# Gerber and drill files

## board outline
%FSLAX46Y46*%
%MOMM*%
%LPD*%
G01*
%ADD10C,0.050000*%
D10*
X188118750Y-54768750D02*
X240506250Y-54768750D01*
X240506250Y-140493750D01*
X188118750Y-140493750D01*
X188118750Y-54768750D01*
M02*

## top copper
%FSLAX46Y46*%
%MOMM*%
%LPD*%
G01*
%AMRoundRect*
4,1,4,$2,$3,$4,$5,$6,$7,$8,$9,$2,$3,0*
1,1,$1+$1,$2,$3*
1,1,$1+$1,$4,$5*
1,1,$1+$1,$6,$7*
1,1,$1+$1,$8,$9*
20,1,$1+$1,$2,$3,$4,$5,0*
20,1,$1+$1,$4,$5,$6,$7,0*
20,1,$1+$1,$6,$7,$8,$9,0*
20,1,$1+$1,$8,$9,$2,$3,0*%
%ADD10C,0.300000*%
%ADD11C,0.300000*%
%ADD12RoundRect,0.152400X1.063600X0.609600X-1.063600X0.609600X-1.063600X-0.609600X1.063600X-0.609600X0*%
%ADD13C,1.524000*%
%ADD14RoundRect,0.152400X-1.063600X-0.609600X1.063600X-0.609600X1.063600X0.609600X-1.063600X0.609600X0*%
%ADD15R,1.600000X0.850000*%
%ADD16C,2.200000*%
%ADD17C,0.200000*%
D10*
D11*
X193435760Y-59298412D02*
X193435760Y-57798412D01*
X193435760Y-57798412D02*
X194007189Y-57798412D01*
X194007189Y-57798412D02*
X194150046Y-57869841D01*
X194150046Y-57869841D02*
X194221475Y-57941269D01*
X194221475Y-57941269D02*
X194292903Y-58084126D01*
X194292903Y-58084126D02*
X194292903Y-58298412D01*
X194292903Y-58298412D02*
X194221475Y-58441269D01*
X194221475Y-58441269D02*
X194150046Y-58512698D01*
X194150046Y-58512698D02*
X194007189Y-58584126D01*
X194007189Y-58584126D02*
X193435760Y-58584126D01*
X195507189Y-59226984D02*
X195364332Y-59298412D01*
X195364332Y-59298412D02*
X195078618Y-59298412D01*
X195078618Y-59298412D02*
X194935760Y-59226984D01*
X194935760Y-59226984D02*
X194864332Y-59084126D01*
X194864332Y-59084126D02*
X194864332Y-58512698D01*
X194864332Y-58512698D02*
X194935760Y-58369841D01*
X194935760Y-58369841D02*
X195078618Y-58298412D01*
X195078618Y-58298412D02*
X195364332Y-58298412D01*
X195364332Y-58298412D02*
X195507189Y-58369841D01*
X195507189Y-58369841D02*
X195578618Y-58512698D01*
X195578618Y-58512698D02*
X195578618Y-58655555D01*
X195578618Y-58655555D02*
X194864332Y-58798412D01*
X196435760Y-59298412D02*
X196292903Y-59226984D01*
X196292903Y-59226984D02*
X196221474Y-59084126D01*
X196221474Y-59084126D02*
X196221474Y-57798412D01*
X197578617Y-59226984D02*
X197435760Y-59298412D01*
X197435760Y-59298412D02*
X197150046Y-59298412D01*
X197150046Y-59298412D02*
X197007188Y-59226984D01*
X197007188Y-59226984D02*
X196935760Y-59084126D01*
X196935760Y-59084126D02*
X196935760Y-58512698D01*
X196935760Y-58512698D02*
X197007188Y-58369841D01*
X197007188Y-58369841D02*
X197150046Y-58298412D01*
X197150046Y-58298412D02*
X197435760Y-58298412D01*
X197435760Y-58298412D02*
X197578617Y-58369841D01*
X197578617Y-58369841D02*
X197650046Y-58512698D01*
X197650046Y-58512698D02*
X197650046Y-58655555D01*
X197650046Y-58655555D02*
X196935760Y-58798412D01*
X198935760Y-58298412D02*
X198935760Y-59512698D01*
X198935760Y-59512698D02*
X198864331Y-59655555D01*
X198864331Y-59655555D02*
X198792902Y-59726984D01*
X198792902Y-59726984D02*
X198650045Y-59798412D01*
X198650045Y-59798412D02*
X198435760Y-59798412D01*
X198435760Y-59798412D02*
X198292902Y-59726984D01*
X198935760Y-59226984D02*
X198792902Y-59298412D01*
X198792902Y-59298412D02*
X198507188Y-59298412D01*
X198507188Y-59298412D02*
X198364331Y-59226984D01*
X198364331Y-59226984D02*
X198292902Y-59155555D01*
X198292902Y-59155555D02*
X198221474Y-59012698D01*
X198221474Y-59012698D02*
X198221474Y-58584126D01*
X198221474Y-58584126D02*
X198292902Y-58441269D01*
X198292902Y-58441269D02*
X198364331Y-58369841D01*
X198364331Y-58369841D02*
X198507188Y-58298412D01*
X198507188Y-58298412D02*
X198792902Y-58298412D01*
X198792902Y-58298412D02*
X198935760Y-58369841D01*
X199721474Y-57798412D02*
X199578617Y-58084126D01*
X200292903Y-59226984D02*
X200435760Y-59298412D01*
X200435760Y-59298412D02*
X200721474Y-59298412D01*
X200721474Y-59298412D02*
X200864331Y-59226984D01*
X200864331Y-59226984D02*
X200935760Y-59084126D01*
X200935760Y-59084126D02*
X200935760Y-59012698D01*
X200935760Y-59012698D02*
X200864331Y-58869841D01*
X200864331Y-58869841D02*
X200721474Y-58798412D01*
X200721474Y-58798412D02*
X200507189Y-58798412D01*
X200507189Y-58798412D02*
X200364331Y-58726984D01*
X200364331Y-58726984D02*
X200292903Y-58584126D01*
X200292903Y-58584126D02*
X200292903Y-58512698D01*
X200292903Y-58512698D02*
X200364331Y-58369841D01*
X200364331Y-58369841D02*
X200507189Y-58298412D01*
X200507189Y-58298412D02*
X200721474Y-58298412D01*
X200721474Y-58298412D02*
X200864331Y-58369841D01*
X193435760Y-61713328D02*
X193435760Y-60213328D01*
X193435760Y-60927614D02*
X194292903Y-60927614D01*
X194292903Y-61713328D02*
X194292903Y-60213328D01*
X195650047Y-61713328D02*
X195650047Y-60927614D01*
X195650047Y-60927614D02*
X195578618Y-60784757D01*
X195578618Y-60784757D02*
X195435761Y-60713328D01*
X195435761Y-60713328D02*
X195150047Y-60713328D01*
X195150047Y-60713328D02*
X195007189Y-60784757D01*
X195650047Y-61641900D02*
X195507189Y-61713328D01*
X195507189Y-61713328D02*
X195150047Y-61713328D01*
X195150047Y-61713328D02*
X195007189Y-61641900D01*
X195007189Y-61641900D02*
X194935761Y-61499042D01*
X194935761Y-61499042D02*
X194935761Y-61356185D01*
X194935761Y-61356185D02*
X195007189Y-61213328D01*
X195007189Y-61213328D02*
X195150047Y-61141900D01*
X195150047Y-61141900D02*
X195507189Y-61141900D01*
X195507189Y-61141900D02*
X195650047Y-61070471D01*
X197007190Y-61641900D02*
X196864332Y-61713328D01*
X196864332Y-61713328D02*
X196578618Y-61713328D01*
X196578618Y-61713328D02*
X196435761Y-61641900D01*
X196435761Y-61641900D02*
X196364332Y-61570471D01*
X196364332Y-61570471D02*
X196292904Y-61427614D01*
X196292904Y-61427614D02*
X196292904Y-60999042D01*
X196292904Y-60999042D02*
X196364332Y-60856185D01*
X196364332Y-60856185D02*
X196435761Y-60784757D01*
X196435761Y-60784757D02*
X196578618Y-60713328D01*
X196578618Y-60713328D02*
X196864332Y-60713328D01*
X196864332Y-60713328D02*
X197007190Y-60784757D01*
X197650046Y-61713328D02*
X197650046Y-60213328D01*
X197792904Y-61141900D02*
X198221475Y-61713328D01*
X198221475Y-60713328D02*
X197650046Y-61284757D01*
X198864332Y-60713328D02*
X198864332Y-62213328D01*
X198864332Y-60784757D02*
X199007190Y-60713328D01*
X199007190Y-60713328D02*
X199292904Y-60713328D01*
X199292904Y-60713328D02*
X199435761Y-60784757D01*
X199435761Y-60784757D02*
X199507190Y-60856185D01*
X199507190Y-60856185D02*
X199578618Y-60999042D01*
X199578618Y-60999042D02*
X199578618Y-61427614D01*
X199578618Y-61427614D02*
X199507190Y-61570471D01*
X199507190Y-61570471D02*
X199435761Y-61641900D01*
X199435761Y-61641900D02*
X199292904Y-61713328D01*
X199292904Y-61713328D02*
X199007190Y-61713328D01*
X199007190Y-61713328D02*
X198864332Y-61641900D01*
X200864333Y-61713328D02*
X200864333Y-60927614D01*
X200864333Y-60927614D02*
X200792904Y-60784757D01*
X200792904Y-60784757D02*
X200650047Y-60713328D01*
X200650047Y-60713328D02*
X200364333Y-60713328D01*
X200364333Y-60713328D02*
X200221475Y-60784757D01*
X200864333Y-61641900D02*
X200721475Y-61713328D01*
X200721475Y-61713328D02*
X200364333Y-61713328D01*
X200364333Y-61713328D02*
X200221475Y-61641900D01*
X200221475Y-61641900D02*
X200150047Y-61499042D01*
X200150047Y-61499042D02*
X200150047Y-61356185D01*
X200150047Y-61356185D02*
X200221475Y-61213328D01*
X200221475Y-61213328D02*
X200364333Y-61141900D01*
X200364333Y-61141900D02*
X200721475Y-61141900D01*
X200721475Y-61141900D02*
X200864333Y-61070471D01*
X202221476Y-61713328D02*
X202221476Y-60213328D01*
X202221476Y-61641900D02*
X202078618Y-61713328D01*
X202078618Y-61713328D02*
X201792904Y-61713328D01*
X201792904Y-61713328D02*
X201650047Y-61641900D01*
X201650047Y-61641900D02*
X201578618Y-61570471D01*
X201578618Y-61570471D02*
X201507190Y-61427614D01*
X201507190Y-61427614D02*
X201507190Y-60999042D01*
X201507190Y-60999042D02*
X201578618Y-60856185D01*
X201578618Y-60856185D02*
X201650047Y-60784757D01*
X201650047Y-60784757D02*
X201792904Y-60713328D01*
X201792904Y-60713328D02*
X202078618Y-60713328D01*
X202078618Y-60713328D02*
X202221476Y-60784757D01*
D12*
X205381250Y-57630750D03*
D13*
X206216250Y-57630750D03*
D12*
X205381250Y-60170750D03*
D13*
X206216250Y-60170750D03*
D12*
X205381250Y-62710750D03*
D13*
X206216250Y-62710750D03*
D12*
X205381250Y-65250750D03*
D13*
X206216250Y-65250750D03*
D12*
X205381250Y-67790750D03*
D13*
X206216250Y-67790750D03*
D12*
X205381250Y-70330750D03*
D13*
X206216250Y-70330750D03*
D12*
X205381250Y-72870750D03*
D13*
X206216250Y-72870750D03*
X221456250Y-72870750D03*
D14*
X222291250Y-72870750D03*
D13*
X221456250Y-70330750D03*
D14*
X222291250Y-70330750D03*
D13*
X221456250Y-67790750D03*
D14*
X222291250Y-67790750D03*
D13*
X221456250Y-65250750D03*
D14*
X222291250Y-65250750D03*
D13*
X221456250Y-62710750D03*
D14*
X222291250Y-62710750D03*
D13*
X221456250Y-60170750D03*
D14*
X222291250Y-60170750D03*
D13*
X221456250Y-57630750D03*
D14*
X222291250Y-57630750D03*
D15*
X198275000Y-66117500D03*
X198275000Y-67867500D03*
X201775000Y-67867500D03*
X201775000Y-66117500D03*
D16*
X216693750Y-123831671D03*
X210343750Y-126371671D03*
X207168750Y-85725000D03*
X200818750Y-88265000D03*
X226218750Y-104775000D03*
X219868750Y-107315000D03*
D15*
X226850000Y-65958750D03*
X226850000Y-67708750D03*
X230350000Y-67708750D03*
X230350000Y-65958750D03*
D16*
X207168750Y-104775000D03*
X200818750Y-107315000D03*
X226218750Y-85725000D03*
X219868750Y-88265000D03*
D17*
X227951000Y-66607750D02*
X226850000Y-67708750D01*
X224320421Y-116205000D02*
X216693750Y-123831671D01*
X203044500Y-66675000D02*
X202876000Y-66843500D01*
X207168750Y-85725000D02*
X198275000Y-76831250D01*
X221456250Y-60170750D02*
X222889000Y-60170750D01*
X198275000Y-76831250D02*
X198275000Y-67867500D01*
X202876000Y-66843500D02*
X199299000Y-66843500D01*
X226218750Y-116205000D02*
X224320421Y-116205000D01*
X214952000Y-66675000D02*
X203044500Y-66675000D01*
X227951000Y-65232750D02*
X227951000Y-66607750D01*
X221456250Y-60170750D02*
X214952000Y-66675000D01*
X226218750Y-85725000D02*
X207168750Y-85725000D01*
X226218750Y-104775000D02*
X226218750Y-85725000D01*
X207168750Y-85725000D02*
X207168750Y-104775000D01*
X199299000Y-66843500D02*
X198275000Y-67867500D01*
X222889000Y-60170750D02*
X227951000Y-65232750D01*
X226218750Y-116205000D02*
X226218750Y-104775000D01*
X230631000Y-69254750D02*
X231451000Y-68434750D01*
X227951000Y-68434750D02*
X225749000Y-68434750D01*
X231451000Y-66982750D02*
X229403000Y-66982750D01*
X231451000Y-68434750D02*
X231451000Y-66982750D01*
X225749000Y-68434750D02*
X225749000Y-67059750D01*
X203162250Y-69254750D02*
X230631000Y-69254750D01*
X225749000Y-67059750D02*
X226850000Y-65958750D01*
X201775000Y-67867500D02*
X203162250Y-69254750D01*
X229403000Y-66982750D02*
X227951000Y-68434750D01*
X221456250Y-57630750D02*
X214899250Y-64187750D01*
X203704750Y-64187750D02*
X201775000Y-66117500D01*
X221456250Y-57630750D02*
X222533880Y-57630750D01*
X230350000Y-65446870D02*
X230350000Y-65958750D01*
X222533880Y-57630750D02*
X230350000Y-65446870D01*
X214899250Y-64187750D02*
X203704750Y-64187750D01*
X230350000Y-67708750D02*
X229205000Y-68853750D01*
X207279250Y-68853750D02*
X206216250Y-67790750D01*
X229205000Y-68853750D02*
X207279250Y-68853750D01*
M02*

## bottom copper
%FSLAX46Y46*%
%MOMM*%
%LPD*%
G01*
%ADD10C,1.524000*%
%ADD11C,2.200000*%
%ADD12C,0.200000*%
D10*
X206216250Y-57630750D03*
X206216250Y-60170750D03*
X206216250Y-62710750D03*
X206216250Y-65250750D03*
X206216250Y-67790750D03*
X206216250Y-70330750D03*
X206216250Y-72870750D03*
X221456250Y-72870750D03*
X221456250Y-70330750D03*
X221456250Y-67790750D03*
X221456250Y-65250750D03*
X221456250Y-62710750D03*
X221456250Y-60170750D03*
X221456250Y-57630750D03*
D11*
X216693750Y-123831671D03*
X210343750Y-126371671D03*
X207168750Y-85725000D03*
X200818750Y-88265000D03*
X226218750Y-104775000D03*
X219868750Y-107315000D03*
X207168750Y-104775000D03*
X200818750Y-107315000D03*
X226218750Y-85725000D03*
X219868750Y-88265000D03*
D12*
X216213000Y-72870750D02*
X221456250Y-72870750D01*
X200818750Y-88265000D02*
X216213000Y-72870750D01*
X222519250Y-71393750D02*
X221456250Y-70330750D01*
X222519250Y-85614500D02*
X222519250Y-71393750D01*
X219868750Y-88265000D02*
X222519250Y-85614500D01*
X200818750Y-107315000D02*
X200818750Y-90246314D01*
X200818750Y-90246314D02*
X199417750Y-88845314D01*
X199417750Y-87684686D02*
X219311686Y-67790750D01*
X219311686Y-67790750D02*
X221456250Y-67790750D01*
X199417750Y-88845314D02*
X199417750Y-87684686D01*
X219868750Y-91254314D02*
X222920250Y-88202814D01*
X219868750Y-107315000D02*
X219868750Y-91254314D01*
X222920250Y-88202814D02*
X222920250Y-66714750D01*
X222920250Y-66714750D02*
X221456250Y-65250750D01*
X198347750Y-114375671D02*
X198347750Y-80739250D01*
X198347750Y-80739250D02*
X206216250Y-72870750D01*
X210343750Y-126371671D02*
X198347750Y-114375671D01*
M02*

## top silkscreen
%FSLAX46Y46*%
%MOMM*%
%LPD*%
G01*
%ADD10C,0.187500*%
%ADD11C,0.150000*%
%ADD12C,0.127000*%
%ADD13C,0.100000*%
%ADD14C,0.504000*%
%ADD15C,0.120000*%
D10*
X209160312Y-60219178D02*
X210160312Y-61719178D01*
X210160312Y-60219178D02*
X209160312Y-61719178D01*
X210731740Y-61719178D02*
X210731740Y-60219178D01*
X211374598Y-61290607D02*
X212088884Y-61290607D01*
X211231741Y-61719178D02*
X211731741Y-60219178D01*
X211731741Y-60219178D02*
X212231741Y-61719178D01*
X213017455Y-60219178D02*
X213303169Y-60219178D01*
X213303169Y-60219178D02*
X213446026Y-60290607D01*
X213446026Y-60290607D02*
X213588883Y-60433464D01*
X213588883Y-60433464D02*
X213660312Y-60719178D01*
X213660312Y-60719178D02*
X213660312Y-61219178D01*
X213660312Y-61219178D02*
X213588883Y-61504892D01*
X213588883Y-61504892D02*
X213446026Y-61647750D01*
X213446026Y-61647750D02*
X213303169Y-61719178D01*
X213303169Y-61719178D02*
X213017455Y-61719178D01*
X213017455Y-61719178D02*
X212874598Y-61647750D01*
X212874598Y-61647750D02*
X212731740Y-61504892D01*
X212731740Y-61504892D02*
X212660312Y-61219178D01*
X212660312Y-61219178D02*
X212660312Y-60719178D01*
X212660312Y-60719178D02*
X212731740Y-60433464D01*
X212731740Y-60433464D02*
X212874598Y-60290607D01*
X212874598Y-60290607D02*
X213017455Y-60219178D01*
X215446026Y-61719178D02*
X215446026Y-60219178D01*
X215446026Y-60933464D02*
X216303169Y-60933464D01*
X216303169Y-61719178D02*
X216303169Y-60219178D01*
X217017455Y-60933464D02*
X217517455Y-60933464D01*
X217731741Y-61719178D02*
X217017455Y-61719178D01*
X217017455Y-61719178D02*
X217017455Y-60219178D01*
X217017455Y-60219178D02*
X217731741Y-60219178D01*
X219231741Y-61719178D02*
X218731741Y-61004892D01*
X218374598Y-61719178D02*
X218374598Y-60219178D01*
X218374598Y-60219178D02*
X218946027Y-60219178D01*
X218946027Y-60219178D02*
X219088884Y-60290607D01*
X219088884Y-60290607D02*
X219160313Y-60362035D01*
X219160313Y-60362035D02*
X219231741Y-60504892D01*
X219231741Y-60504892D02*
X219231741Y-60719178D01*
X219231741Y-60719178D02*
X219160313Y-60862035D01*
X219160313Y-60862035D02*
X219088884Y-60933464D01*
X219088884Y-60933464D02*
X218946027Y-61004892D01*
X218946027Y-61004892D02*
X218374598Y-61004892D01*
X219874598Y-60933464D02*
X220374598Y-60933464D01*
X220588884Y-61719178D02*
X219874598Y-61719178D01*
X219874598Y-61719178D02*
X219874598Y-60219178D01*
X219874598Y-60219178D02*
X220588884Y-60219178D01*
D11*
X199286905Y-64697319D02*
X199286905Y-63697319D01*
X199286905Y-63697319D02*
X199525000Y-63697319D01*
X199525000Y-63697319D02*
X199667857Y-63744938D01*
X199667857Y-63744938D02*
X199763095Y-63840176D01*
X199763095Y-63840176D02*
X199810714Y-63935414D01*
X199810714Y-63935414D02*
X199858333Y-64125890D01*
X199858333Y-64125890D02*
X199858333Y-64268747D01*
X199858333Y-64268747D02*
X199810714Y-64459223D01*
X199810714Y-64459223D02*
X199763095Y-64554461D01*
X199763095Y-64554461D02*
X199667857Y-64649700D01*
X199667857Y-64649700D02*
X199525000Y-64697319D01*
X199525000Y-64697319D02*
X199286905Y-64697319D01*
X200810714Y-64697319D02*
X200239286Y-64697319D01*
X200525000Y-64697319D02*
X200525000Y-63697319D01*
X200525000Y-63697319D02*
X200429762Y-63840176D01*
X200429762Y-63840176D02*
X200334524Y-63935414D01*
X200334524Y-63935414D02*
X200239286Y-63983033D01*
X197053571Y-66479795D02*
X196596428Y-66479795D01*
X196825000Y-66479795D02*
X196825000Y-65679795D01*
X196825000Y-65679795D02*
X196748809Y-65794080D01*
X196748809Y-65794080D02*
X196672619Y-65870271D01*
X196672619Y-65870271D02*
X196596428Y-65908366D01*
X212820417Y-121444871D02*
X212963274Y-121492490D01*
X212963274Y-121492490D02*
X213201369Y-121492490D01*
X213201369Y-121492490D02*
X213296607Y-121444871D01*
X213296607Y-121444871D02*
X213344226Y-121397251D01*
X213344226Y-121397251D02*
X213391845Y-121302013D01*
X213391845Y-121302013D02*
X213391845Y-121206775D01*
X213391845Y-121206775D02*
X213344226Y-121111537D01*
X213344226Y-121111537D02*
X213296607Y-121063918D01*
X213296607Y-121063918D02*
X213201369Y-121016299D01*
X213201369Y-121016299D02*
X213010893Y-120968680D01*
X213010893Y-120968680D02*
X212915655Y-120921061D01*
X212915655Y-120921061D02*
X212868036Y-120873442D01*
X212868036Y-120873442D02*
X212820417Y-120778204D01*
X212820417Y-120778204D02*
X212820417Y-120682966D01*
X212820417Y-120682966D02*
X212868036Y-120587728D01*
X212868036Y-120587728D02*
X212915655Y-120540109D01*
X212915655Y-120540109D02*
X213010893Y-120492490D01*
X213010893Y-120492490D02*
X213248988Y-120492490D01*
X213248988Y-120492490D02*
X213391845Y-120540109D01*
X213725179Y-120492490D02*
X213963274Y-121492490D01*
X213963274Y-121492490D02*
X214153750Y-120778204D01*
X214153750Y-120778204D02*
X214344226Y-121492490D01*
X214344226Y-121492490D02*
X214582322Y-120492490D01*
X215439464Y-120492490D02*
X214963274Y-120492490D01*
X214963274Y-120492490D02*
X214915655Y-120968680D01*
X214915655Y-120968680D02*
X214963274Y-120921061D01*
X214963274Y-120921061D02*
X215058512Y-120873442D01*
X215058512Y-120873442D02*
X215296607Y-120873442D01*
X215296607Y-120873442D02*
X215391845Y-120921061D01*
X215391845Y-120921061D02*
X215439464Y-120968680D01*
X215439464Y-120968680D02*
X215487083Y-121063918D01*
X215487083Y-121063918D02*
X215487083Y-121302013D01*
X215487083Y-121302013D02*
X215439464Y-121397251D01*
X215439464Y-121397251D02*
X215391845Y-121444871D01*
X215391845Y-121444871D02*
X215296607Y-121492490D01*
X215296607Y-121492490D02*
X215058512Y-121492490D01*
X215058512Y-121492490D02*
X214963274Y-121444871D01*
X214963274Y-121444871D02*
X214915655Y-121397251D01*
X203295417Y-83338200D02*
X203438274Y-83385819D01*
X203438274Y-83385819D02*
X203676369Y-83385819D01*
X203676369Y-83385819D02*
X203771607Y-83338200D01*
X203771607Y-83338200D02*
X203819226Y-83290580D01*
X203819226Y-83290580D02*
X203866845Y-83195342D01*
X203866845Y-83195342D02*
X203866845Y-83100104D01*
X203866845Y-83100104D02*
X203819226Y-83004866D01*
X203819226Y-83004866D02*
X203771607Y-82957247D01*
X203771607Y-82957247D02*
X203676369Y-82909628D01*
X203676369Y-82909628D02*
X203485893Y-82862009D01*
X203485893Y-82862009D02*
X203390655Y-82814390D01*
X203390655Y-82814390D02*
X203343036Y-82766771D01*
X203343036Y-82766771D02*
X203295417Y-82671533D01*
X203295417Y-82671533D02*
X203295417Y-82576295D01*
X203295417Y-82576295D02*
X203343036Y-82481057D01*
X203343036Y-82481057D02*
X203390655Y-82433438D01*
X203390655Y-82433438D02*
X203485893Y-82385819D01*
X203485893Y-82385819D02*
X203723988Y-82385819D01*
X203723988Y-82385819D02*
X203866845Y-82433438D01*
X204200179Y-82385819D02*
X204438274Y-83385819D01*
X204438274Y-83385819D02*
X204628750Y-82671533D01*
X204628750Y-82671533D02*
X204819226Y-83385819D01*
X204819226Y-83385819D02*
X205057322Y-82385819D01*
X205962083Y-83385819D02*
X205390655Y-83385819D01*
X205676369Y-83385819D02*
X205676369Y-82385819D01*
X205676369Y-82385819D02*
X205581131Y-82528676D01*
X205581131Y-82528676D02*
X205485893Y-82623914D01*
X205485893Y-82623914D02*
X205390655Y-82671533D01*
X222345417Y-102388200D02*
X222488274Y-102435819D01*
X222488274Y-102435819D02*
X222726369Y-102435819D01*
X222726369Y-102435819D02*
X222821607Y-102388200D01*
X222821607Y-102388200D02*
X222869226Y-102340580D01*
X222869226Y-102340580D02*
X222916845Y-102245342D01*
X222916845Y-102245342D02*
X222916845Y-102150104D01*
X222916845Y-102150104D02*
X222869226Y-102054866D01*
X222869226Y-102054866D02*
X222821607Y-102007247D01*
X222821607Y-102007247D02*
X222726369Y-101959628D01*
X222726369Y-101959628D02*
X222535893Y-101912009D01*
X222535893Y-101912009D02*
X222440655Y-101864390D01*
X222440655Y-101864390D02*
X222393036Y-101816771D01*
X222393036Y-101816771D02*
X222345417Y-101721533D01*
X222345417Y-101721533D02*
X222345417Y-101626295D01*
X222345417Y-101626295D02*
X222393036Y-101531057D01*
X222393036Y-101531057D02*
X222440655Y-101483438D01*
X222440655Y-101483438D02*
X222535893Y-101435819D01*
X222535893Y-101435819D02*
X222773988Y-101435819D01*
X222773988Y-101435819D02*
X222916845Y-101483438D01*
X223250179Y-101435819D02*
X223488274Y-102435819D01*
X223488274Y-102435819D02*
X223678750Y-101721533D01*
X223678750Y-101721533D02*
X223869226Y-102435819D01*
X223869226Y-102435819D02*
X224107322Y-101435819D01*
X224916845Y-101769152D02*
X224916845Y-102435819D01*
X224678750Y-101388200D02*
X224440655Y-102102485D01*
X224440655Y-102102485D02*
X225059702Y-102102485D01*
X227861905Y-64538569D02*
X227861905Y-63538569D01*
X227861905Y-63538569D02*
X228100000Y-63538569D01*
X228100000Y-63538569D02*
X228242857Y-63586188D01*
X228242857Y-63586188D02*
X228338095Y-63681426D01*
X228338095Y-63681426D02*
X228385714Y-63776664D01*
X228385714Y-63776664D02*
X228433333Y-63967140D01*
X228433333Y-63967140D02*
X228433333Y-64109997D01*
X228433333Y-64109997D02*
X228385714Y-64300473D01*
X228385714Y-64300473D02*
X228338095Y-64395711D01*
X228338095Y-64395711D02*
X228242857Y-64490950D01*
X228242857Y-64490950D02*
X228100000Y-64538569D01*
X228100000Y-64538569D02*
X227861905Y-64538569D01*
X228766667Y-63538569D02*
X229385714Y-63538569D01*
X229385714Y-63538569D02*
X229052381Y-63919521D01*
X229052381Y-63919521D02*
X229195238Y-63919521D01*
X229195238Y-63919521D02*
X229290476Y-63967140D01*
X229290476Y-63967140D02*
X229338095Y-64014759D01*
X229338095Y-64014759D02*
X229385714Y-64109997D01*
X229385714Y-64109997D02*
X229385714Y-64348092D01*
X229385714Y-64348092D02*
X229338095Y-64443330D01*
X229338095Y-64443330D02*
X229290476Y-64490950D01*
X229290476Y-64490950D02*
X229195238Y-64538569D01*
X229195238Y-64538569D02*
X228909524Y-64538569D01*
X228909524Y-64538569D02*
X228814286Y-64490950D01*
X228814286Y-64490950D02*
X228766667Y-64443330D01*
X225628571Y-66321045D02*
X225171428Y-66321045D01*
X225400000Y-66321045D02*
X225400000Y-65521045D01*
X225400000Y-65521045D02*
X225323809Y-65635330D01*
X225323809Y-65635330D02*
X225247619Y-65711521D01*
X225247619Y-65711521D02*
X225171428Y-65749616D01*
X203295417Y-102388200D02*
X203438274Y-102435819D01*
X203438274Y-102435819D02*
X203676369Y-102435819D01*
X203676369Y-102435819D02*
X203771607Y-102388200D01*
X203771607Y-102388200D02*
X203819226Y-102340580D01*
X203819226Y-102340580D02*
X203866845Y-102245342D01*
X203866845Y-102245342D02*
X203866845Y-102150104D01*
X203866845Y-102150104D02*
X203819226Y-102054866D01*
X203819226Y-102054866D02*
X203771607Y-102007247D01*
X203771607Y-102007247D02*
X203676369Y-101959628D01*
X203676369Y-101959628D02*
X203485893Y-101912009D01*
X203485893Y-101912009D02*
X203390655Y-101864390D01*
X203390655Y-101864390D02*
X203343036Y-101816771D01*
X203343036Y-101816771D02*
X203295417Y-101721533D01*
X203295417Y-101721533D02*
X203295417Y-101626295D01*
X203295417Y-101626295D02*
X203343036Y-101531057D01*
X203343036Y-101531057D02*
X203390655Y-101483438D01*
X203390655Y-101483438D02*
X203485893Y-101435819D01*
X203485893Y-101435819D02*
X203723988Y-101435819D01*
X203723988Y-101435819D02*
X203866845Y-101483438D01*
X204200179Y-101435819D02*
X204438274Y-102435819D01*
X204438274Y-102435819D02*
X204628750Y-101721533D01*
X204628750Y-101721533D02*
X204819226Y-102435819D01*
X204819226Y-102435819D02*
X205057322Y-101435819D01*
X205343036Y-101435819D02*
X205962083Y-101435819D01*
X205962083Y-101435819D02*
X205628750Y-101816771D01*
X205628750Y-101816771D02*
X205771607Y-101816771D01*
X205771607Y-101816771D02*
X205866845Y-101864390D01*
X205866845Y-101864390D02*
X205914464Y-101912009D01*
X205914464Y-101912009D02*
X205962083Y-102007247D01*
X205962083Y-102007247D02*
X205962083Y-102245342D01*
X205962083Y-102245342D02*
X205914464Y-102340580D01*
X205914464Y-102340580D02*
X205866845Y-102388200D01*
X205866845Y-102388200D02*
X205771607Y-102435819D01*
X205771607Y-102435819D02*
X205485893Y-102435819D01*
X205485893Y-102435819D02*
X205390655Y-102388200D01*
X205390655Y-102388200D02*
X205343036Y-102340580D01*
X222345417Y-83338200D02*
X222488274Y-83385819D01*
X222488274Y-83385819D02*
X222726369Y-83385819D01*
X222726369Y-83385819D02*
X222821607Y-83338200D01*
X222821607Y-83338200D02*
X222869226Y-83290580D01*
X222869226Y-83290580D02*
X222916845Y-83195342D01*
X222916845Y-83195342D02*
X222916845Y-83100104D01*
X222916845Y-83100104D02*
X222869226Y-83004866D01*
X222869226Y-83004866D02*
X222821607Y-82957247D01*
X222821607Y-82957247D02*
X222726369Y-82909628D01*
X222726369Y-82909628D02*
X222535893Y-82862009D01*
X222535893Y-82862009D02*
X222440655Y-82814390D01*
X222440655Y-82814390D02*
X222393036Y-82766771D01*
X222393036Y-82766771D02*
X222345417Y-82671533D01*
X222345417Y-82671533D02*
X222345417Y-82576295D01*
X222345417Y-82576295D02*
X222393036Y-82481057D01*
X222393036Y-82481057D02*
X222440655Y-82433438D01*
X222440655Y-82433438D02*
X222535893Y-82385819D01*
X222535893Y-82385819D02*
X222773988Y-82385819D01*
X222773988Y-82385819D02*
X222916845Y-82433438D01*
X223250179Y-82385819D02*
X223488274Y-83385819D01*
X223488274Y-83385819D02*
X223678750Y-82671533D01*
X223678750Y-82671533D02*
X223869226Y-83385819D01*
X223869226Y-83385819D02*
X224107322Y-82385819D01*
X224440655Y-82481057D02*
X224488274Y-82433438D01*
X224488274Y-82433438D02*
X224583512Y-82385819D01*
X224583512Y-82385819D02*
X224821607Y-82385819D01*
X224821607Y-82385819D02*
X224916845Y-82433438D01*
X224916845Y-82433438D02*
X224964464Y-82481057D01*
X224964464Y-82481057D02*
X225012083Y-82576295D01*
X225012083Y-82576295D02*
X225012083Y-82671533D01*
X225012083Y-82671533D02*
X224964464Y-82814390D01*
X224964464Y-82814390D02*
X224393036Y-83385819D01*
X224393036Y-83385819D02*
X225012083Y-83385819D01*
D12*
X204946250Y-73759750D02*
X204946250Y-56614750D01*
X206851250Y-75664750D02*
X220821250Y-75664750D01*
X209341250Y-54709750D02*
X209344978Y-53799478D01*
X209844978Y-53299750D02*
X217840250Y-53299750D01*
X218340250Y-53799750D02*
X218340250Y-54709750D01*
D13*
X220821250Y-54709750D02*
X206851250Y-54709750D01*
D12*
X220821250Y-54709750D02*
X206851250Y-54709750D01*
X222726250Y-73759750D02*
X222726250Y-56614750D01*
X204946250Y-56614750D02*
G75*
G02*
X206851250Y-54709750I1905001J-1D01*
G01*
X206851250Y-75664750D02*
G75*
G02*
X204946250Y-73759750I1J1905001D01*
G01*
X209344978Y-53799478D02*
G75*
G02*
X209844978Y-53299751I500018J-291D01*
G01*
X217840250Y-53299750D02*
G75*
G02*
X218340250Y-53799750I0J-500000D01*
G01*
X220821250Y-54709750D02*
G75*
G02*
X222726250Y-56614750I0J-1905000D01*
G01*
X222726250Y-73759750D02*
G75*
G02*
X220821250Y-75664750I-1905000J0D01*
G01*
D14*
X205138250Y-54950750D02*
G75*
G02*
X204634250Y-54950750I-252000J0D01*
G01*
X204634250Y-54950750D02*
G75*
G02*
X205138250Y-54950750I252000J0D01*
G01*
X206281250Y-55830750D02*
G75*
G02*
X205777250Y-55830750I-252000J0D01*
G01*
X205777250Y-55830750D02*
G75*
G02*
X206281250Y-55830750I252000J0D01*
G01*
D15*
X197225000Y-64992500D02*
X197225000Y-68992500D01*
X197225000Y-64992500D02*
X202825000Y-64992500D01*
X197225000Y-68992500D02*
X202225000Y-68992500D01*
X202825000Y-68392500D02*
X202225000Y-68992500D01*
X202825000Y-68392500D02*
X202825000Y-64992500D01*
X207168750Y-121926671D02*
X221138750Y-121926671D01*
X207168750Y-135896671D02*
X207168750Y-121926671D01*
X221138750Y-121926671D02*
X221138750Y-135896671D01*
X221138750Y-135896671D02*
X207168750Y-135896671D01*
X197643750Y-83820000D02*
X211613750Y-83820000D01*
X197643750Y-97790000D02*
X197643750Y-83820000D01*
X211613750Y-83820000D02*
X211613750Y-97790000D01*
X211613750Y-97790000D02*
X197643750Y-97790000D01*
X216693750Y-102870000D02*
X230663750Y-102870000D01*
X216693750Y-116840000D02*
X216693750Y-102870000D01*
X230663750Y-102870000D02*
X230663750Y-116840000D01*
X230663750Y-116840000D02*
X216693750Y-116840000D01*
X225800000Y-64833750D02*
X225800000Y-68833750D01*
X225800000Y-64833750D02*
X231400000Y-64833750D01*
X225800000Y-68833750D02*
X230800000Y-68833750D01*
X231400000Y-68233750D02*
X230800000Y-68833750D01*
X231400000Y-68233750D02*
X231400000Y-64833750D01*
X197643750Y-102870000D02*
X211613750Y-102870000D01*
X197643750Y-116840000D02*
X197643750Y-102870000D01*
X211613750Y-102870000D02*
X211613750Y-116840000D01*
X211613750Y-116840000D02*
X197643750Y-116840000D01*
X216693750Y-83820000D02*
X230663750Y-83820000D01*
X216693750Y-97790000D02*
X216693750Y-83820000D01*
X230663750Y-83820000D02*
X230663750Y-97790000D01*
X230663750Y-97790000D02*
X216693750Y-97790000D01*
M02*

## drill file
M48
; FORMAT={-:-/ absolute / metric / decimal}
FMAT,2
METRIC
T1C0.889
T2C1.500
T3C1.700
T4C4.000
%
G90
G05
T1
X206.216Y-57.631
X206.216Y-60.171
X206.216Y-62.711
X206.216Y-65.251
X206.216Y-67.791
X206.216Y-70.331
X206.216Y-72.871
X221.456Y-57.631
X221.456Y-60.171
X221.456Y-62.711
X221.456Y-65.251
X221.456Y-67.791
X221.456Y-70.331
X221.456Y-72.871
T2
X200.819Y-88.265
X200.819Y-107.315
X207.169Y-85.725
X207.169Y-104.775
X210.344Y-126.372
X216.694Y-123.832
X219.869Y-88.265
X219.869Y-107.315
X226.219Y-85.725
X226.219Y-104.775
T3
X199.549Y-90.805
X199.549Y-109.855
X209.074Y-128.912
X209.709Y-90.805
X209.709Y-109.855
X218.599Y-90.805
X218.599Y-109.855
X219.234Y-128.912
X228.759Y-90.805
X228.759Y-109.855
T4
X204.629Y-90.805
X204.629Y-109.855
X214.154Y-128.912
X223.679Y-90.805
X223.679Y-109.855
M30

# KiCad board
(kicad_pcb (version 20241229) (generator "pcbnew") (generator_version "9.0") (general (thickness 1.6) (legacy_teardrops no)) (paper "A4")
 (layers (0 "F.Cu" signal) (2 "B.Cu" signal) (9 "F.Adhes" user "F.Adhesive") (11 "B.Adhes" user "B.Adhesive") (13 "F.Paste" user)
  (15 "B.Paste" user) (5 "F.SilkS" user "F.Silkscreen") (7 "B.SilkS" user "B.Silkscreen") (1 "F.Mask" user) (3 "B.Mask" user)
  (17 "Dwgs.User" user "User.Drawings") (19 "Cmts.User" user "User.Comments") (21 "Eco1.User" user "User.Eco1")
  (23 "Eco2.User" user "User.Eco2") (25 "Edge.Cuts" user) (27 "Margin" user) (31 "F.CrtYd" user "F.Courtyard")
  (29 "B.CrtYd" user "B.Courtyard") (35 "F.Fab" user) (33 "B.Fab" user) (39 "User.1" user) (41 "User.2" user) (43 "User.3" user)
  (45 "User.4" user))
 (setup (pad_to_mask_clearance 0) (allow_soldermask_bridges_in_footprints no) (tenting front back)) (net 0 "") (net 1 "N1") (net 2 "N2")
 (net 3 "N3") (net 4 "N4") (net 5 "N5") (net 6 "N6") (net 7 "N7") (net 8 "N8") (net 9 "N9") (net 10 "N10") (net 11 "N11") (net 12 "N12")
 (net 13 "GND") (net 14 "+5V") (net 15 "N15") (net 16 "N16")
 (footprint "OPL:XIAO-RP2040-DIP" (layer "F.Cu") (at 213.83625 65.25075)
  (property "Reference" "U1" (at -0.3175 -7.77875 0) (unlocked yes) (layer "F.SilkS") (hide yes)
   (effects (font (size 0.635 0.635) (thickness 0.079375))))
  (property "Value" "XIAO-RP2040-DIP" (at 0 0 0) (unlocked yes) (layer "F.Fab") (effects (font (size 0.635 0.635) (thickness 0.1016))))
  (fp_line (start -8.89 8.509) (end -8.89 -8.636) (stroke (width 0.127) (type solid)) (layer "F.SilkS"))
  (fp_line (start -6.985 10.414) (end 6.985 10.414) (stroke (width 0.127) (type solid)) (layer "F.SilkS"))
  (fp_line (start -4.495 -10.541) (end -4.491272 -11.451272) (stroke (width 0.127) (type solid)) (layer "F.SilkS"))
  (fp_line (start -3.991272 -11.951) (end 4.004 -11.951) (stroke (width 0.127) (type solid)) (layer "F.SilkS"))
  (fp_line (start 4.504 -11.451) (end 4.504 -10.541) (stroke (width 0.127) (type solid)) (layer "F.SilkS"))
  (fp_line (start 6.985 -10.541) (end -6.985 -10.541) (stroke (width 0.1) (type solid)) (layer "F.SilkS"))
  (fp_line (start 6.985 -10.541) (end -6.985 -10.541) (stroke (width 0.127) (type solid)) (layer "F.SilkS"))
  (fp_line (start 8.89 8.509) (end 8.89 -8.636) (stroke (width 0.127) (type solid)) (layer "F.SilkS"))
  (fp_arc (start -8.89 -8.636) (mid -8.332038 -9.983038) (end -6.985 -10.541) (stroke (width 0.127) (type solid)) (layer "F.SilkS"))
  (fp_arc (start -6.985 10.414) (mid -8.332038 9.856038) (end -8.89 8.509) (stroke (width 0.127) (type solid)) (layer "F.SilkS"))
  (fp_arc (start -4.491272 -11.451272) (mid -4.344728 -11.80464) (end -3.991272 -11.951) (stroke (width 0.127) (type default))
   (layer "F.SilkS"))
  (fp_arc (start 4.004 -11.951) (mid 4.357553 -11.804553) (end 4.504 -11.451) (stroke (width 0.127) (type default)) (layer "F.SilkS"))
  (fp_arc (start 6.985 -10.541) (mid 8.332038 -9.983038) (end 8.89 -8.636) (stroke (width 0.127) (type solid)) (layer "F.SilkS"))
  (fp_arc (start 8.89 8.509) (mid 8.332038 9.856038) (end 6.985 10.414) (stroke (width 0.127) (type solid)) (layer "F.SilkS"))
  (fp_circle (center -8.95 -10.3) (end -8.95 -10.554) (stroke (width 0.5) (type solid)) (fill yes) (layer "F.SilkS"))
  (fp_circle (center -7.807 -9.42) (end -7.807 -9.674) (stroke (width 0.5) (type solid)) (fill yes) (layer "F.SilkS"))
  (pad "1" smd roundrect (at -8.455 -7.62 180) (size 2.432 1.524) (layers "F.Cu" "F.Mask") (roundrect_rratio 0.1) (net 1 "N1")
   (thermal_bridge_angle 45))
  (pad "1" thru_hole circle (at -7.62 -7.62 180) (size 1.524 1.524) (drill 0.889) (layers "*.Cu" "*.Mask") (remove_unused_layers no)
   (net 1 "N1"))
  (pad "2" smd roundrect (at -8.455 -5.08 180) (size 2.432 1.524) (layers "F.Cu" "F.Mask") (roundrect_rratio 0.1) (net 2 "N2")
   (thermal_bridge_angle 45))
  (pad "2" thru_hole circle (at -7.62 -5.08 180) (size 1.524 1.524) (drill 0.889) (layers "*.Cu" "*.Mask") (remove_unused_layers no)
   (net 2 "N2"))
  (pad "3" smd roundrect (at -8.455 -2.54 180) (size 2.432 1.524) (layers "F.Cu" "F.Mask") (roundrect_rratio 0.1) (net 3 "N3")
   (thermal_bridge_angle 45))
  (pad "3" thru_hole circle (at -7.62 -2.54 180) (size 1.524 1.524) (drill 0.889) (layers "*.Cu" "*.Mask") (remove_unused_layers no)
   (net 3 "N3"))
  (pad "4" smd roundrect (at -8.455 0 180) (size 2.432 1.524) (layers "F.Cu" "F.Mask") (roundrect_rratio 0.1) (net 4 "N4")
   (thermal_bridge_angle 45))
  (pad "4" thru_hole circle (at -7.62 0 180) (size 1.524 1.524) (drill 0.889) (layers "*.Cu" "*.Mask") (remove_unused_layers no)
   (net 4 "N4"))
  (pad "5" smd roundrect (at -8.455 2.54 180) (size 2.432 1.524) (layers "F.Cu" "F.Mask") (roundrect_rratio 0.1) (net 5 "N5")
   (thermal_bridge_angle 45))
  (pad "5" thru_hole circle (at -7.62 2.54 180) (size 1.524 1.524) (drill 0.889) (layers "*.Cu" "*.Mask") (remove_unused_layers no)
   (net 5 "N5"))
  (pad "6" smd roundrect (at -8.455 5.08 180) (size 2.432 1.524) (layers "F.Cu" "F.Mask") (roundrect_rratio 0.1) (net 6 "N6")
   (thermal_bridge_angle 45))
  (pad "6" thru_hole circle (at -7.62 5.08 180) (size 1.524 1.524) (drill 0.889) (layers "*.Cu" "*.Mask") (remove_unused_layers no)
   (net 6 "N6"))
  (pad "7" smd roundrect (at -8.455 7.62 180) (size 2.432 1.524) (layers "F.Cu" "F.Mask") (roundrect_rratio 0.1) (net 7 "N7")
   (thermal_bridge_angle 45))
  (pad "7" thru_hole circle (at -7.62 7.62 180) (size 1.524 1.524) (drill 0.889) (layers "*.Cu" "*.Mask") (remove_unused_layers no)
   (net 7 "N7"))
  (pad "8" thru_hole circle (at 7.62 7.62) (size 1.524 1.524) (drill 0.889) (layers "*.Cu" "*.Mask") (remove_unused_layers no) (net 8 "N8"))
  (pad "8" smd roundrect (at 8.455 7.62) (size 2.432 1.524) (layers "F.Cu" "F.Mask") (roundrect_rratio 0.1) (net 8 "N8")
   (thermal_bridge_angle 45))
  (pad "9" thru_hole circle (at 7.62 5.08) (size 1.524 1.524) (drill 0.889) (layers "*.Cu" "*.Mask") (remove_unused_layers no) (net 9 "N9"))
  (pad "9" smd roundrect (at 8.455 5.08) (size 2.432 1.524) (layers "F.Cu" "F.Mask") (roundrect_rratio 0.1) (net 9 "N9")
   (thermal_bridge_angle 45))
  (pad "10" thru_hole circle (at 7.62 2.54) (size 1.524 1.524) (drill 0.889) (layers "*.Cu" "*.Mask") (remove_unused_layers no)
   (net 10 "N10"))
  (pad "10" smd roundrect (at 8.455 2.54) (size 2.432 1.524) (layers "F.Cu" "F.Mask") (roundrect_rratio 0.1) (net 10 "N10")
   (thermal_bridge_angle 45))
  (pad "11" thru_hole circle (at 7.62 0) (size 1.524 1.524) (drill 0.889) (layers "*.Cu" "*.Mask") (remove_unused_layers no) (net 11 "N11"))
  (pad "11" smd roundrect (at 8.455 0) (size 2.432 1.524) (layers "F.Cu" "F.Mask") (roundrect_rratio 0.1) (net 11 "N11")
   (thermal_bridge_angle 45))
  (pad "12" thru_hole circle (at 7.62 -2.54) (size 1.524 1.524) (drill 0.889) (layers "*.Cu" "*.Mask") (remove_unused_layers no)
   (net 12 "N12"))
  (pad "12" smd roundrect (at 8.455 -2.54) (size 2.432 1.524) (layers "F.Cu" "F.Mask") (roundrect_rratio 0.1) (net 12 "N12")
   (thermal_bridge_angle 45))
  (pad "13" thru_hole circle (at 7.62 -5.08) (size 1.524 1.524) (drill 0.889) (layers "*.Cu" "*.Mask") (remove_unused_layers no)
   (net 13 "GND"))
  (pad "13" smd roundrect (at 8.455 -5.08) (size 2.432 1.524) (layers "F.Cu" "F.Mask") (roundrect_rratio 0.1) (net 13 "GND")
   (thermal_bridge_angle 45))
  (pad "14" thru_hole circle (at 7.62 -7.62) (size 1.524 1.524) (drill 0.889) (layers "*.Cu" "*.Mask") (remove_unused_layers no)
   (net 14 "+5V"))
  (pad "14" smd roundrect (at 8.455 -7.62) (size 2.432 1.524) (layers "F.Cu" "F.Mask") (roundrect_rratio 0.1) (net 14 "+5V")
   (thermal_bridge_angle 45)))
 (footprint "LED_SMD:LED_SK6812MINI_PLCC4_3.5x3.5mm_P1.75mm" (layer "F.Cu") (at 200.025 66.9925)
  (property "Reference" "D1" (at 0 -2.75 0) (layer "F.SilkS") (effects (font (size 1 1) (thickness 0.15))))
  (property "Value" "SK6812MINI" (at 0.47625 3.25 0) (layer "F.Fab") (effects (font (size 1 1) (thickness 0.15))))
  (fp_line (start -2.8 -2) (end -2.8 2) (stroke (width 0.12) (type default)) (layer "F.SilkS"))
  (fp_line (start -2.8 -2) (end 2.8 -2) (stroke (width 0.12) (type solid)) (layer "F.SilkS"))
  (fp_line (start -2.8 2) (end 2.2 2) (stroke (width 0.12) (type solid)) (layer "F.SilkS"))
  (fp_line (start 2.8 1.4) (end 2.2 2) (stroke (width 0.12) (type default)) (layer "F.SilkS"))
  (fp_line (start 2.8 1.4) (end 2.8 -2) (stroke (width 0.12) (type solid)) (layer "F.SilkS"))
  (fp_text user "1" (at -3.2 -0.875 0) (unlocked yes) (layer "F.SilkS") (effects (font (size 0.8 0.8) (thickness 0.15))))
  (pad "1" smd rect (at -1.75 -0.875) (size 1.6 0.85) (layers "F.Cu" "F.Mask" "F.Paste") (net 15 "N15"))
  (pad "2" smd rect (at -1.75 0.875) (size 1.6 0.85) (layers "F.Cu" "F.Mask" "F.Paste") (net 13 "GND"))
  (pad "3" smd rect (at 1.75 0.875) (size 1.6 0.85) (layers "F.Cu" "F.Mask" "F.Paste") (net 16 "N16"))
  (pad "4" smd rect (at 1.75 -0.875) (size 1.6 0.85) (layers "F.Cu" "F.Mask" "F.Paste") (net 14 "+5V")))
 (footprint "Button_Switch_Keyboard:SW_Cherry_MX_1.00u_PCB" (layer "F.Cu") (at 216.69375 123.831671)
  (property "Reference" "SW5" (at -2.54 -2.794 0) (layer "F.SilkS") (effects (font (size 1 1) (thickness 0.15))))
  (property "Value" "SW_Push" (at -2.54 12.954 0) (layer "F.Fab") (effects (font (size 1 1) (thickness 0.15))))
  (fp_line (start -9.525 -1.905) (end 4.445 -1.905) (stroke (width 0.12) (type solid)) (layer "F.SilkS"))
  (fp_line (start -9.525 12.065) (end -9.525 -1.905) (stroke (width 0.12) (type solid)) (layer "F.SilkS"))
  (fp_line (start 4.445 -1.905) (end 4.445 12.065) (stroke (width 0.12) (type solid)) (layer "F.SilkS"))
  (fp_line (start 4.445 12.065) (end -9.525 12.065) (stroke (width 0.12) (type solid)) (layer "F.SilkS"))
  (pad "" np_thru_hole circle (at -7.62 5.08) (size 1.7 1.7) (drill 1.7) (layers "*.Cu" "*.Mask"))
  (pad "" np_thru_hole circle (at -2.54 5.08) (size 4 4) (drill 4) (layers "*.Cu" "*.Mask"))
  (pad "" np_thru_hole circle (at 2.54 5.08) (size 1.7 1.7) (drill 1.7) (layers "*.Cu" "*.Mask"))
  (pad "1" thru_hole circle (at 0 0) (size 2.2 2.2) (drill 1.5) (layers "*.Cu" "*.Mask") (remove_unused_layers no) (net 13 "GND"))
  (pad "2" thru_hole circle (at -6.35 2.54) (size 2.2 2.2) (drill 1.5) (layers "*.Cu" "*.Mask") (remove_unused_layers no) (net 7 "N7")))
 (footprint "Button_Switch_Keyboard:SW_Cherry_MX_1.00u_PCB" (layer "F.Cu") (at 207.16875 85.725)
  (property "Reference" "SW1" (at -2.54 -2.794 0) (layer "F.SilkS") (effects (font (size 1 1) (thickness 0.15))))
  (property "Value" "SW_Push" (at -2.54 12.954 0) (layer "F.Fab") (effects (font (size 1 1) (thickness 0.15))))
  (fp_line (start -9.525 -1.905) (end 4.445 -1.905) (stroke (width 0.12) (type solid)) (layer "F.SilkS"))
  (fp_line (start -9.525 12.065) (end -9.525 -1.905) (stroke (width 0.12) (type solid)) (layer "F.SilkS"))
  (fp_line (start 4.445 -1.905) (end 4.445 12.065) (stroke (width 0.12) (type solid)) (layer "F.SilkS"))
  (fp_line (start 4.445 12.065) (end -9.525 12.065) (stroke (width 0.12) (type solid)) (layer "F.SilkS"))
  (pad "" np_thru_hole circle (at -7.62 5.08) (size 1.7 1.7) (drill 1.7) (layers "*.Cu" "*.Mask"))
  (pad "" np_thru_hole circle (at -2.54 5.08) (size 4 4) (drill 4) (layers "*.Cu" "*.Mask"))
  (pad "" np_thru_hole circle (at 2.54 5.08) (size 1.7 1.7) (drill 1.7) (layers "*.Cu" "*.Mask"))
  (pad "1" thru_hole circle (at 0 0) (size 2.2 2.2) (drill 1.5) (layers "*.Cu" "*.Mask") (remove_unused_layers no) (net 13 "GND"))
  (pad "2" thru_hole circle (at -6.35 2.54) (size 2.2 2.2) (drill 1.5) (layers "*.Cu" "*.Mask") (remove_unused_layers no) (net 8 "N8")))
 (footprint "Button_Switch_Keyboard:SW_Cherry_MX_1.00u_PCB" (layer "F.Cu") (at 226.21875 104.775)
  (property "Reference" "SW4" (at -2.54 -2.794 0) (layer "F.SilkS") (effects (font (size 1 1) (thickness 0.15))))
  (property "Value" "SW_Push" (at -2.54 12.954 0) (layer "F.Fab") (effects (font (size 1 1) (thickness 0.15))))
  (fp_line (start -9.525 -1.905) (end 4.445 -1.905) (stroke (width 0.12) (type solid)) (layer "F.SilkS"))
  (fp_line (start -9.525 12.065) (end -9.525 -1.905) (stroke (width 0.12) (type solid)) (layer "F.SilkS"))
  (fp_line (start 4.445 -1.905) (end 4.445 12.065) (stroke (width 0.12) (type solid)) (layer "F.SilkS"))
  (fp_line (start 4.445 12.065) (end -9.525 12.065) (stroke (width 0.12) (type solid)) (layer "F.SilkS"))
  (pad "" np_thru_hole circle (at -7.62 5.08) (size 1.7 1.7) (drill 1.7) (layers "*.Cu" "*.Mask"))
  (pad "" np_thru_hole circle (at -2.54 5.08) (size 4 4) (drill 4) (layers "*.Cu" "*.Mask"))
  (pad "" np_thru_hole circle (at 2.54 5.08) (size 1.7 1.7) (drill 1.7) (layers "*.Cu" "*.Mask"))
  (pad "1" thru_hole circle (at 0 0) (size 2.2 2.2) (drill 1.5) (layers "*.Cu" "*.Mask") (remove_unused_layers no) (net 13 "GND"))
  (pad "2" thru_hole circle (at -6.35 2.54) (size 2.2 2.2) (drill 1.5) (layers "*.Cu" "*.Mask") (remove_unused_layers no) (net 11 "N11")))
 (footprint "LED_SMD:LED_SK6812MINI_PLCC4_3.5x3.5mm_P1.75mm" (layer "F.Cu") (at 228.6 66.83375)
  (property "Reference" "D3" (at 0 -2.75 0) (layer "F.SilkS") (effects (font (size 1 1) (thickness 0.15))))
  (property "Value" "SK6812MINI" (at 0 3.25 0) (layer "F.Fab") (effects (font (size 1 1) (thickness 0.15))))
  (fp_line (start -2.8 -2) (end -2.8 2) (stroke (width 0.12) (type default)) (layer "F.SilkS"))
  (fp_line (start -2.8 -2) (end 2.8 -2) (stroke (width 0.12) (type solid)) (layer "F.SilkS"))
  (fp_line (start -2.8 2) (end 2.2 2) (stroke (width 0.12) (type solid)) (layer "F.SilkS"))
  (fp_line (start 2.8 1.4) (end 2.2 2) (stroke (width 0.12) (type default)) (layer "F.SilkS"))
  (fp_line (start 2.8 1.4) (end 2.8 -2) (stroke (width 0.12) (type solid)) (layer "F.SilkS"))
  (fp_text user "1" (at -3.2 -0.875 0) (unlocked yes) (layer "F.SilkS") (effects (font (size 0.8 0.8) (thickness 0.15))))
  (pad "1" smd rect (at -1.75 -0.875) (size 1.6 0.85) (layers "F.Cu" "F.Mask" "F.Paste") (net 16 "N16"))
  (pad "2" smd rect (at -1.75 0.875) (size 1.6 0.85) (layers "F.Cu" "F.Mask" "F.Paste") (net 13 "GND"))
  (pad "3" smd rect (at 1.75 0.875) (size 1.6 0.85) (layers "F.Cu" "F.Mask" "F.Paste") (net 5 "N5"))
  (pad "4" smd rect (at 1.75 -0.875) (size 1.6 0.85) (layers "F.Cu" "F.Mask" "F.Paste") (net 14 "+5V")))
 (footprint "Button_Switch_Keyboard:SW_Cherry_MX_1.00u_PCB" (layer "F.Cu") (at 207.16875 104.775)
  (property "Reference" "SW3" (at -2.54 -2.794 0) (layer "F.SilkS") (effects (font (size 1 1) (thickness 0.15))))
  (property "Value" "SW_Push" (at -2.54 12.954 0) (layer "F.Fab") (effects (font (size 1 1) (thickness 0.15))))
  (fp_line (start -9.525 -1.905) (end 4.445 -1.905) (stroke (width 0.12) (type solid)) (layer "F.SilkS"))
  (fp_line (start -9.525 12.065) (end -9.525 -1.905) (stroke (width 0.12) (type solid)) (layer "F.SilkS"))
  (fp_line (start 4.445 -1.905) (end 4.445 12.065) (stroke (width 0.12) (type solid)) (layer "F.SilkS"))
  (fp_line (start 4.445 12.065) (end -9.525 12.065) (stroke (width 0.12) (type solid)) (layer "F.SilkS"))
  (pad "" np_thru_hole circle (at -7.62 5.08) (size 1.7 1.7) (drill 1.7) (layers "*.Cu" "*.Mask"))
  (pad "" np_thru_hole circle (at -2.54 5.08) (size 4 4) (drill 4) (layers "*.Cu" "*.Mask"))
  (pad "" np_thru_hole circle (at 2.54 5.08) (size 1.7 1.7) (drill 1.7) (layers "*.Cu" "*.Mask"))
  (pad "1" thru_hole circle (at 0 0) (size 2.2 2.2) (drill 1.5) (layers "*.Cu" "*.Mask") (remove_unused_layers no) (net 13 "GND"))
  (pad "2" thru_hole circle (at -6.35 2.54) (size 2.2 2.2) (drill 1.5) (layers "*.Cu" "*.Mask") (remove_unused_layers no) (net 10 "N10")))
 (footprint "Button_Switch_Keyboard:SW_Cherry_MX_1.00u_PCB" (layer "F.Cu") (at 226.21875 85.725)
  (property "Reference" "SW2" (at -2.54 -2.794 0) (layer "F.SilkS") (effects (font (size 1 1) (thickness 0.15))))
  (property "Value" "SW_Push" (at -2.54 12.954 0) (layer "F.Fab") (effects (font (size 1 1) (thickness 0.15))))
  (fp_line (start -9.525 -1.905) (end 4.445 -1.905) (stroke (width 0.12) (type solid)) (layer "F.SilkS"))
  (fp_line (start -9.525 12.065) (end -9.525 -1.905) (stroke (width 0.12) (type solid)) (layer "F.SilkS"))
  (fp_line (start 4.445 -1.905) (end 4.445 12.065) (stroke (width 0.12) (type solid)) (layer "F.SilkS"))
  (fp_line (start 4.445 12.065) (end -9.525 12.065) (stroke (width 0.12) (type solid)) (layer "F.SilkS"))
  (pad "" np_thru_hole circle (at -7.62 5.08) (size 1.7 1.7) (drill 1.7) (layers "*.Cu" "*.Mask"))
  (pad "" np_thru_hole circle (at -2.54 5.08) (size 4 4) (drill 4) (layers "*.Cu" "*.Mask"))
  (pad "" np_thru_hole circle (at 2.54 5.08) (size 1.7 1.7) (drill 1.7) (layers "*.Cu" "*.Mask"))
  (pad "1" thru_hole circle (at 0 0) (size 2.2 2.2) (drill 1.5) (layers "*.Cu" "*.Mask") (remove_unused_layers no) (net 13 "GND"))
  (pad "2" thru_hole circle (at -6.35 2.54) (size 2.2 2.2) (drill 1.5) (layers "*.Cu" "*.Mask") (remove_unused_layers no) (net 9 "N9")))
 (gr_rect (start 188.11875 54.76875) (end 240.50625 140.49375) (stroke (width 0.05) (type default)) (fill no) (layer "Edge.Cuts"))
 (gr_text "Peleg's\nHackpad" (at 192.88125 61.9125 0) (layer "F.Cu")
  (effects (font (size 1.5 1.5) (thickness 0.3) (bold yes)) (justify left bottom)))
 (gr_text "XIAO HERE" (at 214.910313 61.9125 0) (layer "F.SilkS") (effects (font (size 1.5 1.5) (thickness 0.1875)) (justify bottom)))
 (segment (start 227.951 66.60775) (end 226.85 67.70875) (width 0.2) (layer "F.Cu") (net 13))
 (segment (start 224.320421 116.205) (end 216.69375 123.831671) (width 0.2) (layer "F.Cu") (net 13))
 (segment (start 203.0445 66.675) (end 202.876 66.8435) (width 0.2) (layer "F.Cu") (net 13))
 (segment (start 207.16875 85.725) (end 198.275 76.83125) (width 0.2) (layer "F.Cu") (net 13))
 (segment (start 221.45625 60.17075) (end 222.889 60.17075) (width 0.2) (layer "F.Cu") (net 13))
 (segment (start 198.275 76.83125) (end 198.275 67.8675) (width 0.2) (layer "F.Cu") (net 13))
 (segment (start 202.876 66.8435) (end 199.299 66.8435) (width 0.2) (layer "F.Cu") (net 13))
 (segment (start 226.21875 116.205) (end 224.320421 116.205) (width 0.2) (layer "F.Cu") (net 13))
 (segment (start 214.952 66.675) (end 203.0445 66.675) (width 0.2) (layer "F.Cu") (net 13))
 (segment (start 227.951 65.23275) (end 227.951 66.60775) (width 0.2) (layer "F.Cu") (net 13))
 (segment (start 221.45625 60.17075) (end 214.952 66.675) (width 0.2) (layer "F.Cu") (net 13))
 (segment (start 226.21875 85.725) (end 207.16875 85.725) (width 0.2) (layer "F.Cu") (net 13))
 (segment (start 226.21875 104.775) (end 226.21875 85.725) (width 0.2) (layer "F.Cu") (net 13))
 (segment (start 207.16875 85.725) (end 207.16875 104.775) (width 0.2) (layer "F.Cu") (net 13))
 (segment (start 199.299 66.8435) (end 198.275 67.8675) (width 0.2) (layer "F.Cu") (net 13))
 (segment (start 222.889 60.17075) (end 227.951 65.23275) (width 0.2) (layer "F.Cu") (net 13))
 (segment (start 226.21875 116.205) (end 226.21875 104.775) (width 0.2) (layer "F.Cu") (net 13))
 (segment (start 230.631 69.25475) (end 231.451 68.43475) (width 0.2) (layer "F.Cu") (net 16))
 (segment (start 227.951 68.43475) (end 225.749 68.43475) (width 0.2) (layer "F.Cu") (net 16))
 (segment (start 231.451 66.98275) (end 229.403 66.98275) (width 0.2) (layer "F.Cu") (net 16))
 (segment (start 231.451 68.43475) (end 231.451 66.98275) (width 0.2) (layer "F.Cu") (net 16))
 (segment (start 225.749 68.43475) (end 225.749 67.05975) (width 0.2) (layer "F.Cu") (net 16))
 (segment (start 203.16225 69.25475) (end 230.631 69.25475) (width 0.2) (layer "F.Cu") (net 16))
 (segment (start 225.749 67.05975) (end 226.85 65.95875) (width 0.2) (layer "F.Cu") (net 16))
 (segment (start 201.775 67.8675) (end 203.16225 69.25475) (width 0.2) (layer "F.Cu") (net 16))
 (segment (start 229.403 66.98275) (end 227.951 68.43475) (width 0.2) (layer "F.Cu") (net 16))
 (segment (start 221.45625 57.63075) (end 214.89925 64.18775) (width 0.2) (layer "F.Cu") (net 14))
 (segment (start 203.70475 64.18775) (end 201.775 66.1175) (width 0.2) (layer "F.Cu") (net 14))
 (segment (start 221.45625 57.63075) (end 222.53388 57.63075) (width 0.2) (layer "F.Cu") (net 14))
 (segment (start 230.35 65.44687) (end 230.35 65.95875) (width 0.2) (layer "F.Cu") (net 14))
 (segment (start 222.53388 57.63075) (end 230.35 65.44687) (width 0.2) (layer "F.Cu") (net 14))
 (segment (start 214.89925 64.18775) (end 203.70475 64.18775) (width 0.2) (layer "F.Cu") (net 14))
 (segment (start 230.35 67.70875) (end 229.205 68.85375) (width 0.2) (layer "F.Cu") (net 5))
 (segment (start 207.27925 68.85375) (end 206.21625 67.79075) (width 0.2) (layer "F.Cu") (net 5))
 (segment (start 229.205 68.85375) (end 207.27925 68.85375) (width 0.2) (layer "F.Cu") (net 5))
 (segment (start 216.213 72.87075) (end 221.45625 72.87075) (width 0.2) (layer "B.Cu") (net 8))
 (segment (start 200.81875 88.265) (end 216.213 72.87075) (width 0.2) (layer "B.Cu") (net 8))
 (segment (start 222.51925 71.39375) (end 221.45625 70.33075) (width 0.2) (layer "B.Cu") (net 9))
 (segment (start 222.51925 85.6145) (end 222.51925 71.39375) (width 0.2) (layer "B.Cu") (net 9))
 (segment (start 219.86875 88.265) (end 222.51925 85.6145) (width 0.2) (layer "B.Cu") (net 9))
 (segment (start 200.81875 107.315) (end 200.81875 90.246314) (width 0.2) (layer "B.Cu") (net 10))
 (segment (start 200.81875 90.246314) (end 199.41775 88.845314) (width 0.2) (layer "B.Cu") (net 10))
 (segment (start 199.41775 87.684686) (end 219.311686 67.79075) (width 0.2) (layer "B.Cu") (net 10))
 (segment (start 219.311686 67.79075) (end 221.45625 67.79075) (width 0.2) (layer "B.Cu") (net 10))
 (segment (start 199.41775 88.845314) (end 199.41775 87.684686) (width 0.2) (layer "B.Cu") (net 10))
 (segment (start 219.86875 91.254314) (end 222.92025 88.202814) (width 0.2) (layer "B.Cu") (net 11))
 (segment (start 219.86875 107.315) (end 219.86875 91.254314) (width 0.2) (layer "B.Cu") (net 11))
 (segment (start 222.92025 88.202814) (end 222.92025 66.71475) (width 0.2) (layer "B.Cu") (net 11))
 (segment (start 222.92025 66.71475) (end 221.45625 65.25075) (width 0.2) (layer "B.Cu") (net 11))
 (segment (start 198.34775 114.375671) (end 198.34775 80.73925) (width 0.2) (layer "B.Cu") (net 7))
 (segment (start 198.34775 80.73925) (end 206.21625 72.87075) (width 0.2) (layer "B.Cu") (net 7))
 (segment (start 210.34375 126.371671) (end 198.34775 114.375671) (width 0.2) (layer "B.Cu") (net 7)))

